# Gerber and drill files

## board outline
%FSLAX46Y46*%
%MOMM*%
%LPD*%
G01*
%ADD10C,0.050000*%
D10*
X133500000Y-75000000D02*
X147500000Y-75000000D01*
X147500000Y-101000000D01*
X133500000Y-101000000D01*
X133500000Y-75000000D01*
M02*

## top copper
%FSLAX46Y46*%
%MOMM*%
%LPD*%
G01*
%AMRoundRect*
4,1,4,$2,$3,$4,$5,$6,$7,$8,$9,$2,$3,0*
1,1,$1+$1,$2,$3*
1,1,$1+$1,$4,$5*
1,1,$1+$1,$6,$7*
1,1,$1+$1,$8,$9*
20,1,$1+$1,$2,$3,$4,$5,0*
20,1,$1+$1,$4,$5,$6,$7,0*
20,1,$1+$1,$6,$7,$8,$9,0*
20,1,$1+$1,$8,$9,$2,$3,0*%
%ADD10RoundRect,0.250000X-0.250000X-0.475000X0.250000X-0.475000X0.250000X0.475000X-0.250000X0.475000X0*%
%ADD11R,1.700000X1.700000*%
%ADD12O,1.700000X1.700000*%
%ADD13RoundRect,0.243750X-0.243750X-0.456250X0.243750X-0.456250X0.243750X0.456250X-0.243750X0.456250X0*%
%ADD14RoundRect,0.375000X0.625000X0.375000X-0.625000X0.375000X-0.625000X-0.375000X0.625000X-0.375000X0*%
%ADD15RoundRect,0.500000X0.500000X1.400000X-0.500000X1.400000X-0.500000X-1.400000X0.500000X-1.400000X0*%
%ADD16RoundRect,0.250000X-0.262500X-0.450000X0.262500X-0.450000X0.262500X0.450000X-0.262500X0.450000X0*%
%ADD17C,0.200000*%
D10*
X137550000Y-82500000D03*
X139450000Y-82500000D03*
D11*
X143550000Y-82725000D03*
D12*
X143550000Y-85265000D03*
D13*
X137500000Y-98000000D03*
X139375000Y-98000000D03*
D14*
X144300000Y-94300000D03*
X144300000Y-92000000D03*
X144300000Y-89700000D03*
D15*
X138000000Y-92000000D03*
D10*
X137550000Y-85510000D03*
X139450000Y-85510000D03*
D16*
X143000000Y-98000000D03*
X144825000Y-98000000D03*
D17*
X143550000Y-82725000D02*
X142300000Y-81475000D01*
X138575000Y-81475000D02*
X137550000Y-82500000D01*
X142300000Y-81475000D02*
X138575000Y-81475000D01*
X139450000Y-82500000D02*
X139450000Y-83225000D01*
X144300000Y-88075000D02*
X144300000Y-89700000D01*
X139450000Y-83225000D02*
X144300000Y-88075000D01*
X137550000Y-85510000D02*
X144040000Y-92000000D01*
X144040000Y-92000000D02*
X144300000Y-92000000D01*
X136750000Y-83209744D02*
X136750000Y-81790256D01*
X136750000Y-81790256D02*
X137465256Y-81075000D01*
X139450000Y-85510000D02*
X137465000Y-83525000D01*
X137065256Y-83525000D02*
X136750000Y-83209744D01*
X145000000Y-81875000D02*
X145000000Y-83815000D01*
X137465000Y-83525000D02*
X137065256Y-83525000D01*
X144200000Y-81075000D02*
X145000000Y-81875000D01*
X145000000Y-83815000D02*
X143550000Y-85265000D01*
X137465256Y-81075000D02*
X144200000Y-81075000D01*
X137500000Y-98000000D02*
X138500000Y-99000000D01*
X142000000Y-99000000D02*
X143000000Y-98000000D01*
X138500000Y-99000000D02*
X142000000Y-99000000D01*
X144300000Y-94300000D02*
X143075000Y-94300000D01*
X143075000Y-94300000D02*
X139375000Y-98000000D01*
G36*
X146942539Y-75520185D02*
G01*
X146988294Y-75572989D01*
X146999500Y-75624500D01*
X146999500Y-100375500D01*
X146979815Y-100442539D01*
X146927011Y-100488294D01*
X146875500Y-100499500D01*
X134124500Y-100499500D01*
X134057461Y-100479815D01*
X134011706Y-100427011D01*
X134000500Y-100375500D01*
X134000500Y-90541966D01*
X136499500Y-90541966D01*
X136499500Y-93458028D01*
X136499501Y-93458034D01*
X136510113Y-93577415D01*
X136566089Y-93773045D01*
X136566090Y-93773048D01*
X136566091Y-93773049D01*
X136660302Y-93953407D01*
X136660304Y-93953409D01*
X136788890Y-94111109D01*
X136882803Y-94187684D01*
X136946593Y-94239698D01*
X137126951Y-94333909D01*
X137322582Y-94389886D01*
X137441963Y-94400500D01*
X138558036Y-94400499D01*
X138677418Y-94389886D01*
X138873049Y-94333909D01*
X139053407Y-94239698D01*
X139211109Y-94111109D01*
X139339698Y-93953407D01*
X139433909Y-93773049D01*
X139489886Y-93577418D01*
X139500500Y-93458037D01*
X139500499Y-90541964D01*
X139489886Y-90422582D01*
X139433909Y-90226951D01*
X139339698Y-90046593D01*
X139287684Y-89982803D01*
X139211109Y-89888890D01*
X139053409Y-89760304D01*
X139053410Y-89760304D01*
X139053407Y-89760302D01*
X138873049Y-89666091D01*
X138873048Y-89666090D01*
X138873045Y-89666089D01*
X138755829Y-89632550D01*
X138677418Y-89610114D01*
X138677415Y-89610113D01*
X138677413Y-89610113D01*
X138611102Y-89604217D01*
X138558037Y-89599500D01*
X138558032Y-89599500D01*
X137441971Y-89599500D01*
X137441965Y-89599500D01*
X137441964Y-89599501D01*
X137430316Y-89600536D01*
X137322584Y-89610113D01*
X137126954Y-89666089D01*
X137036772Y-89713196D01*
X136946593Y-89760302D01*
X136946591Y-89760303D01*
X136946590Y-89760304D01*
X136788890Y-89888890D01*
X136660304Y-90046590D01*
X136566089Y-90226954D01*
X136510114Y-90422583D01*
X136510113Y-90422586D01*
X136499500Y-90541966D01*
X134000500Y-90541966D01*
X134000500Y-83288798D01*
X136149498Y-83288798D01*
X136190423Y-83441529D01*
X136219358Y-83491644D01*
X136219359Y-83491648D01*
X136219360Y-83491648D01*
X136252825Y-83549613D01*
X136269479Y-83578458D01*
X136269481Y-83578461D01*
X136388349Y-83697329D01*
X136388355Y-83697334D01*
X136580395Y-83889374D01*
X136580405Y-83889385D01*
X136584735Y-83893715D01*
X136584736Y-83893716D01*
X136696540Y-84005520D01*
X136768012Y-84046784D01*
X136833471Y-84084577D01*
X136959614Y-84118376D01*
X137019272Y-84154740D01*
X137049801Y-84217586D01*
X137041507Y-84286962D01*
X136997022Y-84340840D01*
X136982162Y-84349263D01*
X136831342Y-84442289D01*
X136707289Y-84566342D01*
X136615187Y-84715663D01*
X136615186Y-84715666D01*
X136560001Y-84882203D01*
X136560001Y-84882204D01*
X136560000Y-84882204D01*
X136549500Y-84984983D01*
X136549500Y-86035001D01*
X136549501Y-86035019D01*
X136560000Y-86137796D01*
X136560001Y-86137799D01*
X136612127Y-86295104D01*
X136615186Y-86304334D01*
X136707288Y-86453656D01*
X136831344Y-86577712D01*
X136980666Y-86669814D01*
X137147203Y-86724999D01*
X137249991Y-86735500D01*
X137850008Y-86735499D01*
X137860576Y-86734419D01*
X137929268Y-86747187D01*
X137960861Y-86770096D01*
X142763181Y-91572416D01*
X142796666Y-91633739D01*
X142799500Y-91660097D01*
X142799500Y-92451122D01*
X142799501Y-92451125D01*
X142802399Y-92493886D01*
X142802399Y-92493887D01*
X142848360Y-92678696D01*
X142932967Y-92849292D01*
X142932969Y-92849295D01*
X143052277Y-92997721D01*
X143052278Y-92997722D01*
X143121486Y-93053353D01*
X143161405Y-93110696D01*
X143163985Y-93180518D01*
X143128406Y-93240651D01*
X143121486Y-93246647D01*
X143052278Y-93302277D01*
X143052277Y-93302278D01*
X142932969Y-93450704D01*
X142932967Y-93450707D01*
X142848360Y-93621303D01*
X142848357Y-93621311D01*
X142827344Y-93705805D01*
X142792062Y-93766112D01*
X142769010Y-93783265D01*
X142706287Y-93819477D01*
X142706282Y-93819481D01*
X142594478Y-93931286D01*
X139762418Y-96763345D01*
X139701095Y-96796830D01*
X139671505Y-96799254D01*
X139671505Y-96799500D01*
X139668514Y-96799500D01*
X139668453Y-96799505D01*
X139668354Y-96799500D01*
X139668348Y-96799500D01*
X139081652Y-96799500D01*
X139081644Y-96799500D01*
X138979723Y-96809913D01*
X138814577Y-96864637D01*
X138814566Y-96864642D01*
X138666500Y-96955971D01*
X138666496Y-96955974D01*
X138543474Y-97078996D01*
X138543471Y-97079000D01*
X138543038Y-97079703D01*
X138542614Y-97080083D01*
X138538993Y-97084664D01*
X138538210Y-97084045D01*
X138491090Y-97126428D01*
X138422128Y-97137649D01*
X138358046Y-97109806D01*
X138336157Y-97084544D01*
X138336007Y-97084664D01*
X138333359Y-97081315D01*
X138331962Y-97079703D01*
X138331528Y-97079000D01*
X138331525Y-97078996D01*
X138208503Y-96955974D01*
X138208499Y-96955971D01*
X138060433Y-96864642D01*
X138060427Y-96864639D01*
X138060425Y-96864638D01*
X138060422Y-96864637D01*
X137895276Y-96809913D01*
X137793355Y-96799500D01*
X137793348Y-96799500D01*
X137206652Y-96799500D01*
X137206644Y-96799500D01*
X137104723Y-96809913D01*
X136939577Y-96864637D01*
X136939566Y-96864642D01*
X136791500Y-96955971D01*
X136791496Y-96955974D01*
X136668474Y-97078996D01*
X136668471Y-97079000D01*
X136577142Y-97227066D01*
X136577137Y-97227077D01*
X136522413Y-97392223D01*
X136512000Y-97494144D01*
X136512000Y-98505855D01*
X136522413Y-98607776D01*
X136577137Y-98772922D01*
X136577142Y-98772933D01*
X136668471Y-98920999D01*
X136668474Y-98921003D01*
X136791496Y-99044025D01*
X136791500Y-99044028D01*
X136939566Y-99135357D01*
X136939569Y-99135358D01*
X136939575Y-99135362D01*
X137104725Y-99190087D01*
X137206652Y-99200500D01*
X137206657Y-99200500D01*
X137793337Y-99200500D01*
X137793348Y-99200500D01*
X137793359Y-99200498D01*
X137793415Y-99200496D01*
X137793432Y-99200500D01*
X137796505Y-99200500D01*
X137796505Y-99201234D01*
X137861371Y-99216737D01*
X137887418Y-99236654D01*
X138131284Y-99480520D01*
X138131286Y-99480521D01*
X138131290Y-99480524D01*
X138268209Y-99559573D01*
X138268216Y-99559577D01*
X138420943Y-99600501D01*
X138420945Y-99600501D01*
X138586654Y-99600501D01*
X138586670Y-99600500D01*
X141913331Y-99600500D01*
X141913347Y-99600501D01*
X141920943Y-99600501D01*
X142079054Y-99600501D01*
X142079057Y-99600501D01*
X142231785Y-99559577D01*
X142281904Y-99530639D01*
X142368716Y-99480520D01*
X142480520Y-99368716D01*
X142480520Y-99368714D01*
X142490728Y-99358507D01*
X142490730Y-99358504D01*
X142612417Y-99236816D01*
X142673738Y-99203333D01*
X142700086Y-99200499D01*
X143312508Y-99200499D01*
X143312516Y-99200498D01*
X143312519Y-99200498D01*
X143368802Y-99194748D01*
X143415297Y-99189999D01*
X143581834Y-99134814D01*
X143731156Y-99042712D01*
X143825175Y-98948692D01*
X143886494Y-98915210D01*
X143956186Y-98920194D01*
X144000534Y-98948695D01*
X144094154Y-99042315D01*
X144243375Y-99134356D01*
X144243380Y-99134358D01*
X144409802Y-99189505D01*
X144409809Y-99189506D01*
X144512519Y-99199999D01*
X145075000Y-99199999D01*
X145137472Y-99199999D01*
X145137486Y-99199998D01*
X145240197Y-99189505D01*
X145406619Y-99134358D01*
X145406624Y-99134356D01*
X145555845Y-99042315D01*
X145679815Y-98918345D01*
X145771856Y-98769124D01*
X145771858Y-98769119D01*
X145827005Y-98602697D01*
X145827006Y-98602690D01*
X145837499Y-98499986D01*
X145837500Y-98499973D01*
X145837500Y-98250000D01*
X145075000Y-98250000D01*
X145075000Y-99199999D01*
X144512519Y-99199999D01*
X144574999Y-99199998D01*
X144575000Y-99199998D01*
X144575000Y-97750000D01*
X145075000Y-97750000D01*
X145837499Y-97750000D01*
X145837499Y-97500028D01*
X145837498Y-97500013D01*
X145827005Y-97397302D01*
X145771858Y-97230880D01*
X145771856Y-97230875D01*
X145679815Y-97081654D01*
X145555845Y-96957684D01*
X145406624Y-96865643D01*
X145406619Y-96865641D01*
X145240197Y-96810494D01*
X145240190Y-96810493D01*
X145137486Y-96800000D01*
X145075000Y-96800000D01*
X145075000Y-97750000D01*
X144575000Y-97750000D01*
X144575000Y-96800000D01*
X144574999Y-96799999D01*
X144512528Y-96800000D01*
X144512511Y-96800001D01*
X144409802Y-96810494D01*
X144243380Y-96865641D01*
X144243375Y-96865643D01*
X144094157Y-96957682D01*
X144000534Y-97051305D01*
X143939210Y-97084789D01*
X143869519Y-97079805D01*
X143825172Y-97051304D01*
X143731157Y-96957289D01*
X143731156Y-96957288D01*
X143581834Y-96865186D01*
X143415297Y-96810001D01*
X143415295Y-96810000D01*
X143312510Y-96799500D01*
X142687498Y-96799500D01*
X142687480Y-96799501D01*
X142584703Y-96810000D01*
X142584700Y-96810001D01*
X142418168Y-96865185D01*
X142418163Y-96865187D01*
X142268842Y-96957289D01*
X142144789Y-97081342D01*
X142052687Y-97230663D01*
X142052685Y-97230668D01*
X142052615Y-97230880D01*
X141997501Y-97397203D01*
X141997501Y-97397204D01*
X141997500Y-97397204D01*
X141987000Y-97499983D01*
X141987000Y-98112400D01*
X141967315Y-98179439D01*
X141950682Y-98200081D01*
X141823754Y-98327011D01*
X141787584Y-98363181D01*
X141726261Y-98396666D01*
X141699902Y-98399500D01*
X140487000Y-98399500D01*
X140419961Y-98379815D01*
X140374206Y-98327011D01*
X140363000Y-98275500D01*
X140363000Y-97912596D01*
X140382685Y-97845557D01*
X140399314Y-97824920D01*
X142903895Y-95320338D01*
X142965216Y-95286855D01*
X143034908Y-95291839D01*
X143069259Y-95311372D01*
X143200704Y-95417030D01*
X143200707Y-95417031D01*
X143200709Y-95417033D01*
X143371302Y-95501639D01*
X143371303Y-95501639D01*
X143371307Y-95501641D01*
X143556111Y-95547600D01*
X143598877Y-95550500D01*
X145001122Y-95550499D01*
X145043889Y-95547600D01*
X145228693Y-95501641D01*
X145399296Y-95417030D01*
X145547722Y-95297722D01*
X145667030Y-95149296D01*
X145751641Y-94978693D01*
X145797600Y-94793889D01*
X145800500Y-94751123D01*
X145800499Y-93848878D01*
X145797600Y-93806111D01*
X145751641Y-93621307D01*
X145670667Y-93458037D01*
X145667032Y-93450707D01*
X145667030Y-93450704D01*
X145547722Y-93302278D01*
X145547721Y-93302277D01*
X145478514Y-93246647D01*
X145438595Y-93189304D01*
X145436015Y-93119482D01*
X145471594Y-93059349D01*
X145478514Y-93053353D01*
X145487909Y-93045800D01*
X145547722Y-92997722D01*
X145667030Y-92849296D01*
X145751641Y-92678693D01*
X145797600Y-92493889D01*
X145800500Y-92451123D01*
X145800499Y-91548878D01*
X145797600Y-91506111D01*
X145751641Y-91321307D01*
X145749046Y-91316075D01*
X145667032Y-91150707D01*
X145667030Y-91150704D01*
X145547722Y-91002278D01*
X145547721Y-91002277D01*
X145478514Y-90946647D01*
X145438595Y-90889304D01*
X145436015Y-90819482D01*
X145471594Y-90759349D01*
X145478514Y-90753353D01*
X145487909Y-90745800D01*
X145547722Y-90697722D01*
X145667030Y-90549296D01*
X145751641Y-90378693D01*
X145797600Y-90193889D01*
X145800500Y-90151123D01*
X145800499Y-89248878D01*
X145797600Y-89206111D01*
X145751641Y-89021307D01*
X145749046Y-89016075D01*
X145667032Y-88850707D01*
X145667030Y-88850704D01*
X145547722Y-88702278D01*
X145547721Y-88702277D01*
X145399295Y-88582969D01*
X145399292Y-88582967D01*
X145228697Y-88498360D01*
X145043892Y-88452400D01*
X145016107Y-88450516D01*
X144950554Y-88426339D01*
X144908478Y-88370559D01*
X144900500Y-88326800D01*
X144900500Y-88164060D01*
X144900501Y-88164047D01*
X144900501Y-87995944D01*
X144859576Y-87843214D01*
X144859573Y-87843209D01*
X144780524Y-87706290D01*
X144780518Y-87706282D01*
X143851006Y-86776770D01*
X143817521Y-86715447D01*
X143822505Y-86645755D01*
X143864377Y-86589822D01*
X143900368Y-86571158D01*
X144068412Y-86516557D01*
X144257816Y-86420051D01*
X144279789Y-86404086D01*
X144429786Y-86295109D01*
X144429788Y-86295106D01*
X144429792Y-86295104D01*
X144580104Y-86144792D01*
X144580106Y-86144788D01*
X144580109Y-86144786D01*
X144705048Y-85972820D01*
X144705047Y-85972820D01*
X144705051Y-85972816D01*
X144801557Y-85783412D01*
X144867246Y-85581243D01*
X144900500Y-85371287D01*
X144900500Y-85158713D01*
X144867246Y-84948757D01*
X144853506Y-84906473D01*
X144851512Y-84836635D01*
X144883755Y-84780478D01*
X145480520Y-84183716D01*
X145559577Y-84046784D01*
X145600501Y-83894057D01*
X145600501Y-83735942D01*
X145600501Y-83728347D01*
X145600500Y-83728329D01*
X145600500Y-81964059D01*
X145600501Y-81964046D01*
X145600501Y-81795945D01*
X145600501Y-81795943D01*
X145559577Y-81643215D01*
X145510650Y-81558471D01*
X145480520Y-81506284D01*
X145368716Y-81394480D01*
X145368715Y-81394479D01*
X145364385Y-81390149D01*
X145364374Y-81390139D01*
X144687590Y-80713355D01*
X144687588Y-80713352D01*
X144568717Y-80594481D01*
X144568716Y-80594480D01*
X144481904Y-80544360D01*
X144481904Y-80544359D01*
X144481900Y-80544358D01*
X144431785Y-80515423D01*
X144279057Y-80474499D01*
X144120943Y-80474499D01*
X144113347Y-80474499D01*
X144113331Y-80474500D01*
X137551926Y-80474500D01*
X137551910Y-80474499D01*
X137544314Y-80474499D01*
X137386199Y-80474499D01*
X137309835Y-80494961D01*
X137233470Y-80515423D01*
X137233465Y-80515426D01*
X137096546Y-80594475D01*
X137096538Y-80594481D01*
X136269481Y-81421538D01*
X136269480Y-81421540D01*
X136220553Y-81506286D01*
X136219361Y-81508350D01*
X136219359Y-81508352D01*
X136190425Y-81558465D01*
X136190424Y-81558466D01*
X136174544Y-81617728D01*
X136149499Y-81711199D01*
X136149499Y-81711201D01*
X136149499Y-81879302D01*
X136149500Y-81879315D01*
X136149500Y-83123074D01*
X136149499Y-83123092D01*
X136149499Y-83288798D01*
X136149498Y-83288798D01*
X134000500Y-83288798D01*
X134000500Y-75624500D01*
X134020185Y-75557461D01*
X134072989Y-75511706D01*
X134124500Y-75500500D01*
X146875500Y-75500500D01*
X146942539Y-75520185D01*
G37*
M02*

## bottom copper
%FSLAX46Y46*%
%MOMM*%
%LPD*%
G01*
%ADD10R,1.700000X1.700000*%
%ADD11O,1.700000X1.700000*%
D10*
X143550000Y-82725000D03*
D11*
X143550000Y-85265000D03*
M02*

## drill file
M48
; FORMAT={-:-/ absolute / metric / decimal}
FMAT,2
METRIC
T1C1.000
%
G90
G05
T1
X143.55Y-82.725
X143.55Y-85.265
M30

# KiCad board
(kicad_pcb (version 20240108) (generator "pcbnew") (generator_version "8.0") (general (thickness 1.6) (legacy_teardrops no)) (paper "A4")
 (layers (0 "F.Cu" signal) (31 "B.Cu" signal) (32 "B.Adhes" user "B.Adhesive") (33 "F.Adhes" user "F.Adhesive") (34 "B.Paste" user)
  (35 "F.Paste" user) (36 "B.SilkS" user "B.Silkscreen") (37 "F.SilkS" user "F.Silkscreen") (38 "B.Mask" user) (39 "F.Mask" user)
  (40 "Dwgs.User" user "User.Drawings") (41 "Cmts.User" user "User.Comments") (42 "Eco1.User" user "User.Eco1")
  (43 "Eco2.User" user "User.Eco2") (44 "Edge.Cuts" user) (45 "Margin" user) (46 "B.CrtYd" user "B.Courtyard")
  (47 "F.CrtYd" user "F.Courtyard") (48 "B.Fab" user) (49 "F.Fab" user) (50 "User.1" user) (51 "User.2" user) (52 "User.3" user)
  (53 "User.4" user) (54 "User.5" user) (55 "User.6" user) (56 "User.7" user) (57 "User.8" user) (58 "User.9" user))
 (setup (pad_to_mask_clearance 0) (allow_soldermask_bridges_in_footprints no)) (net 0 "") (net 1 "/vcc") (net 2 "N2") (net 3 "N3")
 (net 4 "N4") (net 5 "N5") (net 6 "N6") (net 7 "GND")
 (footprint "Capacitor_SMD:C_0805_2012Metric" (layer "F.Cu") (at 138.5 82.5)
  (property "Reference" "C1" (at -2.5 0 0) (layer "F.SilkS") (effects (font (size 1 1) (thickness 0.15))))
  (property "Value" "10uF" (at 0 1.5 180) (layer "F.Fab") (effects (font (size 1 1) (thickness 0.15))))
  (pad "1" smd roundrect (at -0.95 0) (size 1 1.45) (layers "F.Cu" "F.Paste" "F.Mask") (roundrect_rratio 0.25) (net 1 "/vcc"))
  (pad "2" smd roundrect (at 0.95 0) (size 1 1.45) (layers "F.Cu" "F.Paste" "F.Mask") (roundrect_rratio 0.25) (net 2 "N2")))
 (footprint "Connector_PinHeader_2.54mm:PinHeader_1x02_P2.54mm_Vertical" (layer "F.Cu") (at 143.55 82.725)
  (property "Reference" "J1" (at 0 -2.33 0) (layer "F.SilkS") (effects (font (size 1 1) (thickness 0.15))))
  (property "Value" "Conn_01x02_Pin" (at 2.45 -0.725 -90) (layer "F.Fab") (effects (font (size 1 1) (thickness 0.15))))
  (pad "1" thru_hole rect (at 0 0) (size 1.7 1.7) (drill 1) (layers "*.Cu" "*.Mask") (remove_unused_layers no) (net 1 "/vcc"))
  (pad "2" thru_hole oval (at 0 2.54) (size 1.7 1.7) (drill 1) (layers "*.Cu" "*.Mask") (remove_unused_layers no) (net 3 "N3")))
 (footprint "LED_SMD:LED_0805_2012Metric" (layer "F.Cu") (at 138.4375 98)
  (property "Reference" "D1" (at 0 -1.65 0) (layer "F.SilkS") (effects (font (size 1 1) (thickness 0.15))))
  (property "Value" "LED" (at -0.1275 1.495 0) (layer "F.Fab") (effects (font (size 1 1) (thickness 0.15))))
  (pad "1" smd roundrect (at -0.9375 0) (size 0.975 1.4) (layers "F.Cu" "F.Paste" "F.Mask") (roundrect_rratio 0.25) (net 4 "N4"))
  (pad "2" smd roundrect (at 0.9375 0) (size 0.975 1.4) (layers "F.Cu" "F.Paste" "F.Mask") (roundrect_rratio 0.25) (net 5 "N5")))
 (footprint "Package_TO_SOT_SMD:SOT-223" (layer "F.Cu") (at 141.15 92 180)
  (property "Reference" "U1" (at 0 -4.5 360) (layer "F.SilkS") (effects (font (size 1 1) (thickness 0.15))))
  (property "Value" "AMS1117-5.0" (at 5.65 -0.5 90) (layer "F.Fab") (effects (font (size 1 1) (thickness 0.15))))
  (pad "1" smd roundrect (at -3.15 -2.3 180) (size 2 1.5) (layers "F.Cu" "F.Paste" "F.Mask") (roundrect_rratio 0.25) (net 5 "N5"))
  (pad "2" smd roundrect (at -3.15 0 180) (size 2 1.5) (layers "F.Cu" "F.Paste" "F.Mask") (roundrect_rratio 0.25) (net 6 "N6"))
  (pad "3" smd roundrect (at -3.15 2.3 180) (size 2 1.5) (layers "F.Cu" "F.Paste" "F.Mask") (roundrect_rratio 0.25) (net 2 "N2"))
  (pad "4" smd roundrect (at 3.15 0 180) (size 2 3.8) (layers "F.Cu" "F.Paste" "F.Mask") (roundrect_rratio 0.25)))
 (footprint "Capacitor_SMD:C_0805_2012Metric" (layer "F.Cu") (at 138.5 85.51)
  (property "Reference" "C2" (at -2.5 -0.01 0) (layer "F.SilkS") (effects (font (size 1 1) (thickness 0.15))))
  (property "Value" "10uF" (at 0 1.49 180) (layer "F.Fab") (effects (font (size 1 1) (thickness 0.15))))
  (pad "1" smd roundrect (at -0.95 0) (size 1 1.45) (layers "F.Cu" "F.Paste" "F.Mask") (roundrect_rratio 0.25) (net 6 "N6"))
  (pad "2" smd roundrect (at 0.95 0) (size 1 1.45) (layers "F.Cu" "F.Paste" "F.Mask") (roundrect_rratio 0.25) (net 3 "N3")))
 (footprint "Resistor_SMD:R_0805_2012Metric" (layer "F.Cu") (at 143.9125 98)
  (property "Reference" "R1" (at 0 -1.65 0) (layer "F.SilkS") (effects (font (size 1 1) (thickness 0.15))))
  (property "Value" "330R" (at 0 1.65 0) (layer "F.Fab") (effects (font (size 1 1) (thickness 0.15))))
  (pad "1" smd roundrect (at -0.9125 0) (size 1.025 1.4) (layers "F.Cu" "F.Paste" "F.Mask") (roundrect_rratio 0.243902) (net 4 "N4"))
  (pad "2" smd roundrect (at 0.9125 0) (size 1.025 1.4) (layers "F.Cu" "F.Paste" "F.Mask") (roundrect_rratio 0.243902) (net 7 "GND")))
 (gr_rect (start 133.5 75) (end 147.5 101) (stroke (width 0.05) (type default)) (fill none) (layer "Edge.Cuts"))
 (segment (start 143.55 82.725) (end 142.3 81.475) (width 0.2) (layer "F.Cu") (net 1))
 (segment (start 138.575 81.475) (end 137.55 82.5) (width 0.2) (layer "F.Cu") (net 1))
 (segment (start 142.3 81.475) (end 138.575 81.475) (width 0.2) (layer "F.Cu") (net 1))
 (segment (start 139.45 82.5) (end 139.45 83.225) (width 0.2) (layer "F.Cu") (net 2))
 (segment (start 144.3 88.075) (end 144.3 89.7) (width 0.2) (layer "F.Cu") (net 2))
 (segment (start 139.45 83.225) (end 144.3 88.075) (width 0.2) (layer "F.Cu") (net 2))
 (segment (start 137.55 85.51) (end 144.04 92) (width 0.2) (layer "F.Cu") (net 6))
 (segment (start 144.04 92) (end 144.3 92) (width 0.2) (layer "F.Cu") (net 6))
 (segment (start 136.75 83.209744) (end 136.75 81.790256) (width 0.2) (layer "F.Cu") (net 3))
 (segment (start 136.75 81.790256) (end 137.465256 81.075) (width 0.2) (layer "F.Cu") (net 3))
 (segment (start 139.45 85.51) (end 137.465 83.525) (width 0.2) (layer "F.Cu") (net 3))
 (segment (start 137.065256 83.525) (end 136.75 83.209744) (width 0.2) (layer "F.Cu") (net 3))
 (segment (start 145 81.875) (end 145 83.815) (width 0.2) (layer "F.Cu") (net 3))
 (segment (start 137.465 83.525) (end 137.065256 83.525) (width 0.2) (layer "F.Cu") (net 3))
 (segment (start 144.2 81.075) (end 145 81.875) (width 0.2) (layer "F.Cu") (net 3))
 (segment (start 145 83.815) (end 143.55 85.265) (width 0.2) (layer "F.Cu") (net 3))
 (segment (start 137.465256 81.075) (end 144.2 81.075) (width 0.2) (layer "F.Cu") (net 3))
 (segment (start 137.5 98) (end 138.5 99) (width 0.2) (layer "F.Cu") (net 4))
 (segment (start 142 99) (end 143 98) (width 0.2) (layer "F.Cu") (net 4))
 (segment (start 138.5 99) (end 142 99) (width 0.2) (layer "F.Cu") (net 4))
 (segment (start 144.3 94.3) (end 143.075 94.3) (width 0.2) (layer "F.Cu") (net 5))
 (segment (start 143.075 94.3) (end 139.375 98) (width 0.2) (layer "F.Cu") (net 5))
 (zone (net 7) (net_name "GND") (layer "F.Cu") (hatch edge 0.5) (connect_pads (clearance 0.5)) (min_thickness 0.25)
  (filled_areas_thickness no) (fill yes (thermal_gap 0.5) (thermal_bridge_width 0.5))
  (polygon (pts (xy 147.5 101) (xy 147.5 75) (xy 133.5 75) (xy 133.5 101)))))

